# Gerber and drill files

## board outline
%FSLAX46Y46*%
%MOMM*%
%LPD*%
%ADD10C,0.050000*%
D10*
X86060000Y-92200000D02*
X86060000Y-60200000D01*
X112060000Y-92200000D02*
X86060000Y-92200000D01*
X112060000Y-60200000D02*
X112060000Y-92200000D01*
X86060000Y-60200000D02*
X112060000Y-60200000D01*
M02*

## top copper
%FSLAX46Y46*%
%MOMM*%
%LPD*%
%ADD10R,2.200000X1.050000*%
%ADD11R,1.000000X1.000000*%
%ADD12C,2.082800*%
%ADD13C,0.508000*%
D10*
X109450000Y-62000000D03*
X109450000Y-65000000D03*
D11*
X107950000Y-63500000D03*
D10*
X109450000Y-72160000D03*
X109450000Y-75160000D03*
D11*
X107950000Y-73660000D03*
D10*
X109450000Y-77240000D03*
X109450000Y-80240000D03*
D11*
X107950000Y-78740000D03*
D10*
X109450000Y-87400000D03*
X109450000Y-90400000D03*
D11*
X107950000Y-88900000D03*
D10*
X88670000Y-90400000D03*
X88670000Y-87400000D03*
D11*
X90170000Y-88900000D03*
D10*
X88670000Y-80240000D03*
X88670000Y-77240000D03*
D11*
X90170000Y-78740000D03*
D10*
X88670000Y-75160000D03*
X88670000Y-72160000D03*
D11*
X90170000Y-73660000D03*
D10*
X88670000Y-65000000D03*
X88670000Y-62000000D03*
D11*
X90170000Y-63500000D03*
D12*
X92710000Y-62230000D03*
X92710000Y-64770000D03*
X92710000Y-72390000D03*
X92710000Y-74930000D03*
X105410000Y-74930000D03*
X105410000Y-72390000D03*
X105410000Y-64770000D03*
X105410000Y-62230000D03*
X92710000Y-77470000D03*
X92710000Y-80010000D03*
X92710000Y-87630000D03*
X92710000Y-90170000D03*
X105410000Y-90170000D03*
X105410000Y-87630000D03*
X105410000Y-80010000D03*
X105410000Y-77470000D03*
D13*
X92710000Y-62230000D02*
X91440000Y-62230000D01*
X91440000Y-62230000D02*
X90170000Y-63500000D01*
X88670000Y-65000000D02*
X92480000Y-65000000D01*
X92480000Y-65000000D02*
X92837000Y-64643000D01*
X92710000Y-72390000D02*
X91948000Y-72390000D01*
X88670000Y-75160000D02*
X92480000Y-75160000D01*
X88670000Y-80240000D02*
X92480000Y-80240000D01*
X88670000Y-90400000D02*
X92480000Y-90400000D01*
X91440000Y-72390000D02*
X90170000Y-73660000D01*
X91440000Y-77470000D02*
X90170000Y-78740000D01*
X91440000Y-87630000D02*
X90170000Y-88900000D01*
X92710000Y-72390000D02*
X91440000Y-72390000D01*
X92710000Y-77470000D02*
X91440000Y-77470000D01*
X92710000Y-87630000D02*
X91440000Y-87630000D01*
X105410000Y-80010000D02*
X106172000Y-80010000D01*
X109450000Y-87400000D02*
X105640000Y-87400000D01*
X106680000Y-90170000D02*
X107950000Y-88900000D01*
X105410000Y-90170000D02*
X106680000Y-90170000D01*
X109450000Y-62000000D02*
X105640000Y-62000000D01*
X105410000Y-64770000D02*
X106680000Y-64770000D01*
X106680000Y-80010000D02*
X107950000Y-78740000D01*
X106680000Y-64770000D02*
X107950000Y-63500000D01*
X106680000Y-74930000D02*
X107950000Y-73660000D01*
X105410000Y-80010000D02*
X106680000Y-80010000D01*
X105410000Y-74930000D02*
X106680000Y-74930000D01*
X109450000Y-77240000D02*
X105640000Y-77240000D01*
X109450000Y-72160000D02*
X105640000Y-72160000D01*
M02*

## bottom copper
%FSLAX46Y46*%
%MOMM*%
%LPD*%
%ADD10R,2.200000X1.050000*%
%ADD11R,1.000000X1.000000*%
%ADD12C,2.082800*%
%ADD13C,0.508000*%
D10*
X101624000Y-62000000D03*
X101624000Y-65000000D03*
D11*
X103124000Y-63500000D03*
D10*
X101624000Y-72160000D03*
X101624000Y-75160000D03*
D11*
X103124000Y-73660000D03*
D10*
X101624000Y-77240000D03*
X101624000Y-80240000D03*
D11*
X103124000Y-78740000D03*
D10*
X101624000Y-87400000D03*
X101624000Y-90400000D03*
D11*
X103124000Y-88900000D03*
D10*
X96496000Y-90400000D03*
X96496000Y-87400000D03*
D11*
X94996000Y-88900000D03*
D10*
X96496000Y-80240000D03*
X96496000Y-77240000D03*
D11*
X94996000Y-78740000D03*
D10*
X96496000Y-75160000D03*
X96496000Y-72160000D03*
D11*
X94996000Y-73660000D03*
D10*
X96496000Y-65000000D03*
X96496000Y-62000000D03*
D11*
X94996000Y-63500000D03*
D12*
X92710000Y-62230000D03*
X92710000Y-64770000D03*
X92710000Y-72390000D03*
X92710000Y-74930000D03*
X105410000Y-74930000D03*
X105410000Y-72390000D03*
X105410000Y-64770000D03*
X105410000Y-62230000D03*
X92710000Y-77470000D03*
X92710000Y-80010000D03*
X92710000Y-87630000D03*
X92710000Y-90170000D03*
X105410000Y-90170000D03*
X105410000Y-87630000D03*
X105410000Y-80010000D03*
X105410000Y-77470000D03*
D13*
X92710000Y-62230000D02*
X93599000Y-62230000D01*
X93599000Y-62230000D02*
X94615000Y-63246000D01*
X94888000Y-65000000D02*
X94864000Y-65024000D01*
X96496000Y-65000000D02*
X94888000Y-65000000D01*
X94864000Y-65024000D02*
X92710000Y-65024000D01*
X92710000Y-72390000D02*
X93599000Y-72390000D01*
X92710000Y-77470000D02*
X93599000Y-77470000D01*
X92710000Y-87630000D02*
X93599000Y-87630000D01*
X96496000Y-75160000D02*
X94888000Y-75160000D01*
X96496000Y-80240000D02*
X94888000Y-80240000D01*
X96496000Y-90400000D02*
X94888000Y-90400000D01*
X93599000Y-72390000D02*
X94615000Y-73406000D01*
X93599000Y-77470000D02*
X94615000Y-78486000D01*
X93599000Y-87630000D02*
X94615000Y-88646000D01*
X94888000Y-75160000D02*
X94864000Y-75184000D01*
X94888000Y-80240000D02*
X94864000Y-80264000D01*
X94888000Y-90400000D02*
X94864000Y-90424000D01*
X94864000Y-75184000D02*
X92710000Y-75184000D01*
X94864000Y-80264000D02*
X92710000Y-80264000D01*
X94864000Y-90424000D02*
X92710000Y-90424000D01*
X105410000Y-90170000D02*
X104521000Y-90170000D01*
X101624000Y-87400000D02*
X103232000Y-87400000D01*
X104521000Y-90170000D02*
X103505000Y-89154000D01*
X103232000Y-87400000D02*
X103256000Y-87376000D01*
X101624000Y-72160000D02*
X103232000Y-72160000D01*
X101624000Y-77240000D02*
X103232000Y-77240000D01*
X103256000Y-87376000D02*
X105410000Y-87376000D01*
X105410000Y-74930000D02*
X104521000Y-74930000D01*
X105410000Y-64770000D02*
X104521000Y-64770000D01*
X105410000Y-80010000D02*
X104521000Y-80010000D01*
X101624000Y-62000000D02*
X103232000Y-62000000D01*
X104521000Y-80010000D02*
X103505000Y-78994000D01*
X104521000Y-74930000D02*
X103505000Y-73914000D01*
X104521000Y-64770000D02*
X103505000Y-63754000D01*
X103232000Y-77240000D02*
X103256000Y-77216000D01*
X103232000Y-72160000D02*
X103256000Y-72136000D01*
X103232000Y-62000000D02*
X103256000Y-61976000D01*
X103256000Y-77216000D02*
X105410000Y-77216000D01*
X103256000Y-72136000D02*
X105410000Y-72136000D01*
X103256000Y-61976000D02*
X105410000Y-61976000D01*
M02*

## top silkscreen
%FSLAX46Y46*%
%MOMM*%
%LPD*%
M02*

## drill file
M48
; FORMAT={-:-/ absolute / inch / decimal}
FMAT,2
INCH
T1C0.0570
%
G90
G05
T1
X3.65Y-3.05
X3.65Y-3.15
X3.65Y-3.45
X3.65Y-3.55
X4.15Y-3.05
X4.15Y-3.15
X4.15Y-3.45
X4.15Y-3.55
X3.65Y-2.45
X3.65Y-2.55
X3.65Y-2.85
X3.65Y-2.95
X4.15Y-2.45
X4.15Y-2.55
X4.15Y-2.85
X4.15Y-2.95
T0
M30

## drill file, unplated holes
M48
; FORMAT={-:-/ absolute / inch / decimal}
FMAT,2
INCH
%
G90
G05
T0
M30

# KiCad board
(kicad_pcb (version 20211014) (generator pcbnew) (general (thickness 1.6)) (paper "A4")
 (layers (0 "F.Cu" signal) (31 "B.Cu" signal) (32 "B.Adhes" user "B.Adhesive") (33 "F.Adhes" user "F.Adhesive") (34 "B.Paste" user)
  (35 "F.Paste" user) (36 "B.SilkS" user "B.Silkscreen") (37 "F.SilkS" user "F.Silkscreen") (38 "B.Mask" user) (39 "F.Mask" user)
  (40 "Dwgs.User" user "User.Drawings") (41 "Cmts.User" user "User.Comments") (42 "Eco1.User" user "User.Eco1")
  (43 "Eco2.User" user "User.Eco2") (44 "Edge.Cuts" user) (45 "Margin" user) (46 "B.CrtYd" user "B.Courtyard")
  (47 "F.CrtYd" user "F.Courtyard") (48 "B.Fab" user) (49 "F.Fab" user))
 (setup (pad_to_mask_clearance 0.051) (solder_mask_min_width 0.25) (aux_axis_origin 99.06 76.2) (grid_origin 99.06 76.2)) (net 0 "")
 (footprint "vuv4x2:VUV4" (layer "F.Cu") (at 99.06 68.58)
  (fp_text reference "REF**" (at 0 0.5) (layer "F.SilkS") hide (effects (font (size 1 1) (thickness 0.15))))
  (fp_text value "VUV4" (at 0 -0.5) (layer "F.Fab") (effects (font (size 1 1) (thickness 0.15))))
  (pad "A1" thru_hole circle locked (at 6.35 -6.35) (size 2.0828 2.0828) (drill 1.4478) (layers *.Cu *.Mask))
  (pad "A2" thru_hole circle locked (at 6.35 3.81) (size 2.0828 2.0828) (drill 1.4478) (layers *.Cu *.Mask))
  (pad "A3" thru_hole circle locked (at -6.35 6.35) (size 2.0828 2.0828) (drill 1.4478) (layers *.Cu *.Mask))
  (pad "A4" thru_hole circle locked (at -6.35 -3.81) (size 2.0828 2.0828) (drill 1.4478) (layers *.Cu *.Mask))
  (pad "K1" thru_hole circle locked (at 6.35 -3.81) (size 2.0828 2.0828) (drill 1.4478) (layers *.Cu *.Mask))
  (pad "K2" thru_hole circle locked (at 6.35 6.35) (size 2.0828 2.0828) (drill 1.4478) (layers *.Cu *.Mask))
  (pad "K3" thru_hole circle locked (at -6.35 3.81) (size 2.0828 2.0828) (drill 1.4478) (layers *.Cu *.Mask))
  (pad "K4" thru_hole circle locked (at -6.35 -6.35) (size 2.0828 2.0828) (drill 1.4478) (layers *.Cu *.Mask)))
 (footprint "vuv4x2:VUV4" (layer "F.Cu") (at 99.06 83.82)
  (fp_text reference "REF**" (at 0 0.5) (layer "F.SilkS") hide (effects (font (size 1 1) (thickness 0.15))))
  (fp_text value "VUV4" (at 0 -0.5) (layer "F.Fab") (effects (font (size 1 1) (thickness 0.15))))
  (pad "A1" thru_hole circle locked (at 6.35 -6.35) (size 2.0828 2.0828) (drill 1.4478) (layers *.Cu *.Mask))
  (pad "A2" thru_hole circle locked (at 6.35 3.81) (size 2.0828 2.0828) (drill 1.4478) (layers *.Cu *.Mask))
  (pad "A3" thru_hole circle locked (at -6.35 6.35) (size 2.0828 2.0828) (drill 1.4478) (layers *.Cu *.Mask))
  (pad "A4" thru_hole circle locked (at -6.35 -3.81) (size 2.0828 2.0828) (drill 1.4478) (layers *.Cu *.Mask))
  (pad "K1" thru_hole circle locked (at 6.35 -3.81) (size 2.0828 2.0828) (drill 1.4478) (layers *.Cu *.Mask))
  (pad "K2" thru_hole circle locked (at 6.35 6.35) (size 2.0828 2.0828) (drill 1.4478) (layers *.Cu *.Mask))
  (pad "K3" thru_hole circle locked (at -6.35 3.81) (size 2.0828 2.0828) (drill 1.4478) (layers *.Cu *.Mask))
  (pad "K4" thru_hole circle locked (at -6.35 -6.35) (size 2.0828 2.0828) (drill 1.4478) (layers *.Cu *.Mask)))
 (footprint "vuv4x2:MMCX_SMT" (layer "F.Cu") (at 90.17 63.5 90)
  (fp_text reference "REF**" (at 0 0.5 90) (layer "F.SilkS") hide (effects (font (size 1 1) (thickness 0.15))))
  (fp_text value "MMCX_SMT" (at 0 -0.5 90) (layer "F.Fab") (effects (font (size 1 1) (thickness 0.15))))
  (pad "1" smd rect locked (at 0 0 90) (size 1 1) (layers "F.Cu" "F.Paste" "F.Mask"))
  (pad "2" smd rect locked (at -1.5 -1.5 90) (size 1.05 2.2) (layers "F.Cu" "F.Paste" "F.Mask"))
  (pad "2" smd rect locked (at 1.5 -1.5 90) (size 1.05 2.2) (layers "F.Cu" "F.Paste" "F.Mask")))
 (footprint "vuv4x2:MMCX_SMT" (layer "F.Cu") (at 90.17 73.66 90)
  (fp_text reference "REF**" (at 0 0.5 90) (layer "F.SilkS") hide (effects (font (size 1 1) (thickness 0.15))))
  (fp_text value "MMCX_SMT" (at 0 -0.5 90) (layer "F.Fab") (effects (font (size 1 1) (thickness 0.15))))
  (pad "1" smd rect locked (at 0 0 90) (size 1 1) (layers "F.Cu" "F.Paste" "F.Mask"))
  (pad "2" smd rect locked (at 1.5 -1.5 90) (size 1.05 2.2) (layers "F.Cu" "F.Paste" "F.Mask"))
  (pad "2" smd rect locked (at -1.5 -1.5 90) (size 1.05 2.2) (layers "F.Cu" "F.Paste" "F.Mask")))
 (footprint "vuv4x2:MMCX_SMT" (layer "F.Cu") (at 90.17 78.74 90)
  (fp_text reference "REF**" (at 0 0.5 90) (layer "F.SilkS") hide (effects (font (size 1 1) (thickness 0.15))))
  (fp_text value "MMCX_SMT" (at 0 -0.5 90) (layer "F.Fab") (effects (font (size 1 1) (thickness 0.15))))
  (pad "1" smd rect locked (at 0 0 90) (size 1 1) (layers "F.Cu" "F.Paste" "F.Mask"))
  (pad "2" smd rect locked (at -1.5 -1.5 90) (size 1.05 2.2) (layers "F.Cu" "F.Paste" "F.Mask"))
  (pad "2" smd rect locked (at 1.5 -1.5 90) (size 1.05 2.2) (layers "F.Cu" "F.Paste" "F.Mask")))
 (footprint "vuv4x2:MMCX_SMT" (layer "F.Cu") (at 90.17 88.9 90)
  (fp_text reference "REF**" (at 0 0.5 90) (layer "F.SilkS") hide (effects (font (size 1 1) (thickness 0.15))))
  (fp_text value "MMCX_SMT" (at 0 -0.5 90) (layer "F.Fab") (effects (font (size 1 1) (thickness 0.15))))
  (pad "1" smd rect locked (at 0 0 90) (size 1 1) (layers "F.Cu" "F.Paste" "F.Mask"))
  (pad "2" smd rect locked (at -1.5 -1.5 90) (size 1.05 2.2) (layers "F.Cu" "F.Paste" "F.Mask"))
  (pad "2" smd rect locked (at 1.5 -1.5 90) (size 1.05 2.2) (layers "F.Cu" "F.Paste" "F.Mask")))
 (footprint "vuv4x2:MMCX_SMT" (layer "F.Cu") (at 107.95 88.9 -90)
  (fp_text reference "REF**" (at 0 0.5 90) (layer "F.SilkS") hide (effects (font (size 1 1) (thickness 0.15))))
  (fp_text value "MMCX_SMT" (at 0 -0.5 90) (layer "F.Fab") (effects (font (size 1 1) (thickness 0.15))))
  (pad "1" smd rect locked (at 0 0 270) (size 1 1) (layers "F.Cu" "F.Paste" "F.Mask"))
  (pad "2" smd rect locked (at 1.5 -1.5 270) (size 1.05 2.2) (layers "F.Cu" "F.Paste" "F.Mask"))
  (pad "2" smd rect locked (at -1.5 -1.5 270) (size 1.05 2.2) (layers "F.Cu" "F.Paste" "F.Mask")))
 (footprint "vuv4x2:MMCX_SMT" (layer "F.Cu") (at 107.95 78.74 -90)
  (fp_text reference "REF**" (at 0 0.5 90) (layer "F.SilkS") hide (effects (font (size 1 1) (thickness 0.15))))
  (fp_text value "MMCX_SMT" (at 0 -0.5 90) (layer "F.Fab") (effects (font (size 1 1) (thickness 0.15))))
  (pad "1" smd rect locked (at 0 0 270) (size 1 1) (layers "F.Cu" "F.Paste" "F.Mask"))
  (pad "2" smd rect locked (at 1.5 -1.5 270) (size 1.05 2.2) (layers "F.Cu" "F.Paste" "F.Mask"))
  (pad "2" smd rect locked (at -1.5 -1.5 270) (size 1.05 2.2) (layers "F.Cu" "F.Paste" "F.Mask")))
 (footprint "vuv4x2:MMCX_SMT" (layer "F.Cu") (at 107.95 73.66 -90)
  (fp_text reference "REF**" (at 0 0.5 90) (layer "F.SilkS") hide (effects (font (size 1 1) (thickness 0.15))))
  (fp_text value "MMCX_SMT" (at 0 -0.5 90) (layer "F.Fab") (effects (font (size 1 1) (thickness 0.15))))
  (pad "1" smd rect locked (at 0 0 270) (size 1 1) (layers "F.Cu" "F.Paste" "F.Mask"))
  (pad "2" smd rect locked (at -1.5 -1.5 270) (size 1.05 2.2) (layers "F.Cu" "F.Paste" "F.Mask"))
  (pad "2" smd rect locked (at 1.5 -1.5 270) (size 1.05 2.2) (layers "F.Cu" "F.Paste" "F.Mask")))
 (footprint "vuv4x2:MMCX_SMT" (layer "F.Cu") (at 107.95 63.5 -90)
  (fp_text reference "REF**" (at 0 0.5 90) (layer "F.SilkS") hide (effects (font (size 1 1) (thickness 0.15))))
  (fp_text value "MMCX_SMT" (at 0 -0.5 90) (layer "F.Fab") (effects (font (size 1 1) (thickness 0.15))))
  (pad "1" smd rect locked (at 0 0 270) (size 1 1) (layers "F.Cu" "F.Paste" "F.Mask"))
  (pad "2" smd rect locked (at -1.5 -1.5 270) (size 1.05 2.2) (layers "F.Cu" "F.Paste" "F.Mask"))
  (pad "2" smd rect locked (at 1.5 -1.5 270) (size 1.05 2.2) (layers "F.Cu" "F.Paste" "F.Mask")))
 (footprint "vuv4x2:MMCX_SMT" (layer "B.Cu") (at 94.996 63.5 90)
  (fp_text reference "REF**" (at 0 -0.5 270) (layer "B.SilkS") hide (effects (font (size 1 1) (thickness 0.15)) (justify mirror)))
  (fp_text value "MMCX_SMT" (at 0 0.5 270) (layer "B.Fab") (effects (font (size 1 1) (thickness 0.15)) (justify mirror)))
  (pad "1" smd rect locked (at 0 0 90) (size 1 1) (layers "B.Cu" "B.Paste" "B.Mask"))
  (pad "2" smd rect locked (at -1.5 1.5 90) (size 1.05 2.2) (layers "B.Cu" "B.Paste" "B.Mask"))
  (pad "2" smd rect locked (at 1.5 1.5 90) (size 1.05 2.2) (layers "B.Cu" "B.Paste" "B.Mask")))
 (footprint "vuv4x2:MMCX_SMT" (layer "B.Cu") (at 94.996 73.66 90)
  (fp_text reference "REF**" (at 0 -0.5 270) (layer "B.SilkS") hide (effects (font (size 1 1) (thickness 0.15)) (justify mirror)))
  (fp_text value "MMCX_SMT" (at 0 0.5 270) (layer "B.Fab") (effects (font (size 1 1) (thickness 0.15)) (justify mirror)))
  (pad "1" smd rect locked (at 0 0 90) (size 1 1) (layers "B.Cu" "B.Paste" "B.Mask"))
  (pad "2" smd rect locked (at -1.5 1.5 90) (size 1.05 2.2) (layers "B.Cu" "B.Paste" "B.Mask"))
  (pad "2" smd rect locked (at 1.5 1.5 90) (size 1.05 2.2) (layers "B.Cu" "B.Paste" "B.Mask")))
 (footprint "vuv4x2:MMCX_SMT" (layer "B.Cu") (at 94.996 78.74 90)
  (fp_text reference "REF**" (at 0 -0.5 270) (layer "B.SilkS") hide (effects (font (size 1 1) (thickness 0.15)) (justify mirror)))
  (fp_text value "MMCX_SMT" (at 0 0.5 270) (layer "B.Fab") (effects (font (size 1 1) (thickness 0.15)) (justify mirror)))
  (pad "1" smd rect locked (at 0 0 90) (size 1 1) (layers "B.Cu" "B.Paste" "B.Mask"))
  (pad "2" smd rect locked (at -1.5 1.5 90) (size 1.05 2.2) (layers "B.Cu" "B.Paste" "B.Mask"))
  (pad "2" smd rect locked (at 1.5 1.5 90) (size 1.05 2.2) (layers "B.Cu" "B.Paste" "B.Mask")))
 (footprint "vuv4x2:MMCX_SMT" (layer "B.Cu") (at 94.996 88.9 90)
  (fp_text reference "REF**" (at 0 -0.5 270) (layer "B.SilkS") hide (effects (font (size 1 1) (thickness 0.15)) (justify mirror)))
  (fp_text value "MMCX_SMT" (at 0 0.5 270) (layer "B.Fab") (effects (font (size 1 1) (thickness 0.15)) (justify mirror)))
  (pad "1" smd rect locked (at 0 0 90) (size 1 1) (layers "B.Cu" "B.Paste" "B.Mask"))
  (pad "2" smd rect locked (at 1.5 1.5 90) (size 1.05 2.2) (layers "B.Cu" "B.Paste" "B.Mask"))
  (pad "2" smd rect locked (at -1.5 1.5 90) (size 1.05 2.2) (layers "B.Cu" "B.Paste" "B.Mask")))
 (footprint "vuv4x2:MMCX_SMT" (layer "B.Cu") (at 103.124 88.9 -90)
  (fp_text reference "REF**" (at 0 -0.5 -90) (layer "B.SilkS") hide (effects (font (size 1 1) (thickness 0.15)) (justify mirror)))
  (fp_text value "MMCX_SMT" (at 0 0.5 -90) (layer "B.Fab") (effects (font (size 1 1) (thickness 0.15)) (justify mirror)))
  (pad "1" smd rect locked (at 0 0 270) (size 1 1) (layers "B.Cu" "B.Paste" "B.Mask"))
  (pad "2" smd rect locked (at -1.5 1.5 270) (size 1.05 2.2) (layers "B.Cu" "B.Paste" "B.Mask"))
  (pad "2" smd rect locked (at 1.5 1.5 270) (size 1.05 2.2) (layers "B.Cu" "B.Paste" "B.Mask")))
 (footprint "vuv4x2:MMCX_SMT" (layer "B.Cu") (at 103.124 78.74 -90)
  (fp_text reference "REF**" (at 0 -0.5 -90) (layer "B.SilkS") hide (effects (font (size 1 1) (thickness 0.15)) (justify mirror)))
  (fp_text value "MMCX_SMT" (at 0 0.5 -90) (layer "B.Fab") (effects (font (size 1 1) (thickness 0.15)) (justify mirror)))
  (pad "1" smd rect locked (at 0 0 270) (size 1 1) (layers "B.Cu" "B.Paste" "B.Mask"))
  (pad "2" smd rect locked (at -1.5 1.5 270) (size 1.05 2.2) (layers "B.Cu" "B.Paste" "B.Mask"))
  (pad "2" smd rect locked (at 1.5 1.5 270) (size 1.05 2.2) (layers "B.Cu" "B.Paste" "B.Mask")))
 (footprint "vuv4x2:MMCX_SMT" (layer "B.Cu") (at 103.124 73.66 -90)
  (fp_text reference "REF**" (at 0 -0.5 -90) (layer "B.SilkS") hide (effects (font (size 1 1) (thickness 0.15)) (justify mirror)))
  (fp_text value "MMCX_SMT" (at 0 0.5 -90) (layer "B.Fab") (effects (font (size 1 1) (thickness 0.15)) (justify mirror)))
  (pad "1" smd rect locked (at 0 0 270) (size 1 1) (layers "B.Cu" "B.Paste" "B.Mask"))
  (pad "2" smd rect locked (at -1.5 1.5 270) (size 1.05 2.2) (layers "B.Cu" "B.Paste" "B.Mask"))
  (pad "2" smd rect locked (at 1.5 1.5 270) (size 1.05 2.2) (layers "B.Cu" "B.Paste" "B.Mask")))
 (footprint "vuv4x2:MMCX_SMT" (layer "B.Cu") (at 103.124 63.5 -90)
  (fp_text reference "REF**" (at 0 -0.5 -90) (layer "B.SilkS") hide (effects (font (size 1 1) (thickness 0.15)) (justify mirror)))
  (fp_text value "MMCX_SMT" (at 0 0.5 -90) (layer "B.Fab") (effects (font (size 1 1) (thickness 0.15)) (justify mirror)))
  (pad "1" smd rect locked (at 0 0 270) (size 1 1) (layers "B.Cu" "B.Paste" "B.Mask"))
  (pad "2" smd rect locked (at 1.5 1.5 270) (size 1.05 2.2) (layers "B.Cu" "B.Paste" "B.Mask"))
  (pad "2" smd rect locked (at -1.5 1.5 270) (size 1.05 2.2) (layers "B.Cu" "B.Paste" "B.Mask")))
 (gr_line (start 86.06 92.2) (end 86.06 60.2) (layer "Edge.Cuts") (width 0.05))
 (gr_line (start 112.06 92.2) (end 86.06 92.2) (layer "Edge.Cuts") (width 0.05))
 (gr_line (start 112.06 60.2) (end 112.06 92.2) (layer "Edge.Cuts") (width 0.05))
 (gr_line (start 86.06 60.2) (end 112.06 60.2) (layer "Edge.Cuts") (width 0.05))
 (segment (start 88.67 75.16) (end 92.48 75.16) (width 0.508) (layer "F.Cu") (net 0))
 (segment (start 88.67 80.24) (end 92.48 80.24) (width 0.508) (layer "F.Cu") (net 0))
 (segment (start 88.67 90.4) (end 92.48 90.4) (width 0.508) (layer "F.Cu") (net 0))
 (segment (start 91.44 72.39) (end 90.17 73.66) (width 0.508) (layer "F.Cu") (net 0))
 (segment (start 91.44 77.47) (end 90.17 78.74) (width 0.508) (layer "F.Cu") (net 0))
 (segment (start 91.44 87.63) (end 90.17 88.9) (width 0.508) (layer "F.Cu") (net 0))
 (segment (start 92.71 72.39) (end 91.44 72.39) (width 0.508) (layer "F.Cu") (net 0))
 (segment (start 92.71 77.47) (end 91.44 77.47) (width 0.508) (layer "F.Cu") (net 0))
 (segment (start 92.71 87.63) (end 91.44 87.63) (width 0.508) (layer "F.Cu") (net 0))
 (segment (start 105.41 80.01) (end 106.172 80.01) (width 0.508) (layer "F.Cu") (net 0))
 (segment (start 109.45 87.4) (end 105.64 87.4) (width 0.508) (layer "F.Cu") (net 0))
 (segment (start 106.68 90.17) (end 107.95 88.9) (width 0.508) (layer "F.Cu") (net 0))
 (segment (start 105.41 90.17) (end 106.68 90.17) (width 0.508) (layer "F.Cu") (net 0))
 (segment (start 109.45 62) (end 105.64 62) (width 0.508) (layer "F.Cu") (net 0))
 (segment (start 105.41 64.77) (end 106.68 64.77) (width 0.508) (layer "F.Cu") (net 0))
 (segment (start 106.68 80.01) (end 107.95 78.74) (width 0.508) (layer "F.Cu") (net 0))
 (segment (start 106.68 64.77) (end 107.95 63.5) (width 0.508) (layer "F.Cu") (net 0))
 (segment (start 106.68 74.93) (end 107.95 73.66) (width 0.508) (layer "F.Cu") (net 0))
 (segment (start 105.41 80.01) (end 106.68 80.01) (width 0.508) (layer "F.Cu") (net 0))
 (segment (start 105.41 74.93) (end 106.68 74.93) (width 0.508) (layer "F.Cu") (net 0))
 (segment (start 109.45 77.24) (end 105.64 77.24) (width 0.508) (layer "F.Cu") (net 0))
 (segment (start 109.45 72.16) (end 105.64 72.16) (width 0.508) (layer "F.Cu") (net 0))
 (segment (start 91.44 62.23) (end 90.17 63.5) (width 0.508) (layer "F.Cu") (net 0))
 (segment (start 92.71 62.23) (end 91.44 62.23) (width 0.508) (layer "F.Cu") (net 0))
 (segment (start 88.67 65) (end 92.48 65) (width 0.508) (layer "F.Cu") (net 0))
 (segment (start 92.48 65) (end 92.837 64.643) (width 0.508) (layer "F.Cu") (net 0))
 (segment (start 92.71 72.39) (end 91.948 72.39) (width 0.508) (layer "F.Cu") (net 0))
 (segment (start 92.71 72.39) (end 93.599 72.39) (width 0.508) (layer "B.Cu") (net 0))
 (segment (start 92.71 77.47) (end 93.599 77.47) (width 0.508) (layer "B.Cu") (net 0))
 (segment (start 92.71 87.63) (end 93.599 87.63) (width 0.508) (layer "B.Cu") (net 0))
 (segment (start 96.496 75.16) (end 94.888 75.16) (width 0.508) (layer "B.Cu") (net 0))
 (segment (start 96.496 80.24) (end 94.888 80.24) (width 0.508) (layer "B.Cu") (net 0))
 (segment (start 96.496 90.4) (end 94.888 90.4) (width 0.508) (layer "B.Cu") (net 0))
 (segment (start 93.599 72.39) (end 94.615 73.406) (width 0.508) (layer "B.Cu") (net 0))
 (segment (start 93.599 77.47) (end 94.615 78.486) (width 0.508) (layer "B.Cu") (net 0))
 (segment (start 93.599 87.63) (end 94.615 88.646) (width 0.508) (layer "B.Cu") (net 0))
 (segment (start 94.888 75.16) (end 94.864 75.184) (width 0.508) (layer "B.Cu") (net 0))
 (segment (start 94.888 80.24) (end 94.864 80.264) (width 0.508) (layer "B.Cu") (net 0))
 (segment (start 94.888 90.4) (end 94.864 90.424) (width 0.508) (layer "B.Cu") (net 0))
 (segment (start 94.864 75.184) (end 92.71 75.184) (width 0.508) (layer "B.Cu") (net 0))
 (segment (start 94.864 80.264) (end 92.71 80.264) (width 0.508) (layer "B.Cu") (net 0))
 (segment (start 94.864 90.424) (end 92.71 90.424) (width 0.508) (layer "B.Cu") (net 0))
 (segment (start 105.41 90.17) (end 104.521 90.17) (width 0.508) (layer "B.Cu") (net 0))
 (segment (start 101.624 87.4) (end 103.232 87.4) (width 0.508) (layer "B.Cu") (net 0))
 (segment (start 104.521 90.17) (end 103.505 89.154) (width 0.508) (layer "B.Cu") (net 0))
 (segment (start 103.232 87.4) (end 103.256 87.376) (width 0.508) (layer "B.Cu") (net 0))
 (segment (start 101.624 72.16) (end 103.232 72.16) (width 0.508) (layer "B.Cu") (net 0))
 (segment (start 101.624 77.24) (end 103.232 77.24) (width 0.508) (layer "B.Cu") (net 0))
 (segment (start 103.256 87.376) (end 105.41 87.376) (width 0.508) (layer "B.Cu") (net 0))
 (segment (start 105.41 74.93) (end 104.521 74.93) (width 0.508) (layer "B.Cu") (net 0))
 (segment (start 105.41 64.77) (end 104.521 64.77) (width 0.508) (layer "B.Cu") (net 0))
 (segment (start 105.41 80.01) (end 104.521 80.01) (width 0.508) (layer "B.Cu") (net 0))
 (segment (start 101.624 62) (end 103.232 62) (width 0.508) (layer "B.Cu") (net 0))
 (segment (start 104.521 80.01) (end 103.505 78.994) (width 0.508) (layer "B.Cu") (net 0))
 (segment (start 104.521 74.93) (end 103.505 73.914) (width 0.508) (layer "B.Cu") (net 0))
 (segment (start 104.521 64.77) (end 103.505 63.754) (width 0.508) (layer "B.Cu") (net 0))
 (segment (start 103.232 77.24) (end 103.256 77.216) (width 0.508) (layer "B.Cu") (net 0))
 (segment (start 103.232 72.16) (end 103.256 72.136) (width 0.508) (layer "B.Cu") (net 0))
 (segment (start 103.232 62) (end 103.256 61.976) (width 0.508) (layer "B.Cu") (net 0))
 (segment (start 103.256 77.216) (end 105.41 77.216) (width 0.508) (layer "B.Cu") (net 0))
 (segment (start 103.256 72.136) (end 105.41 72.136) (width 0.508) (layer "B.Cu") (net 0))
 (segment (start 103.256 61.976) (end 105.41 61.976) (width 0.508) (layer "B.Cu") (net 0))
 (segment (start 92.71 62.23) (end 93.599 62.23) (width 0.508) (layer "B.Cu") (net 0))
 (segment (start 96.496 65) (end 94.888 65) (width 0.508) (layer "B.Cu") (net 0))
 (segment (start 93.599 62.23) (end 94.615 63.246) (width 0.508) (layer "B.Cu") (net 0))
 (segment (start 94.864 65.024) (end 92.71 65.024) (width 0.508) (layer "B.Cu") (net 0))
 (segment (start 94.888 65) (end 94.864 65.024) (width 0.508) (layer "B.Cu") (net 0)))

